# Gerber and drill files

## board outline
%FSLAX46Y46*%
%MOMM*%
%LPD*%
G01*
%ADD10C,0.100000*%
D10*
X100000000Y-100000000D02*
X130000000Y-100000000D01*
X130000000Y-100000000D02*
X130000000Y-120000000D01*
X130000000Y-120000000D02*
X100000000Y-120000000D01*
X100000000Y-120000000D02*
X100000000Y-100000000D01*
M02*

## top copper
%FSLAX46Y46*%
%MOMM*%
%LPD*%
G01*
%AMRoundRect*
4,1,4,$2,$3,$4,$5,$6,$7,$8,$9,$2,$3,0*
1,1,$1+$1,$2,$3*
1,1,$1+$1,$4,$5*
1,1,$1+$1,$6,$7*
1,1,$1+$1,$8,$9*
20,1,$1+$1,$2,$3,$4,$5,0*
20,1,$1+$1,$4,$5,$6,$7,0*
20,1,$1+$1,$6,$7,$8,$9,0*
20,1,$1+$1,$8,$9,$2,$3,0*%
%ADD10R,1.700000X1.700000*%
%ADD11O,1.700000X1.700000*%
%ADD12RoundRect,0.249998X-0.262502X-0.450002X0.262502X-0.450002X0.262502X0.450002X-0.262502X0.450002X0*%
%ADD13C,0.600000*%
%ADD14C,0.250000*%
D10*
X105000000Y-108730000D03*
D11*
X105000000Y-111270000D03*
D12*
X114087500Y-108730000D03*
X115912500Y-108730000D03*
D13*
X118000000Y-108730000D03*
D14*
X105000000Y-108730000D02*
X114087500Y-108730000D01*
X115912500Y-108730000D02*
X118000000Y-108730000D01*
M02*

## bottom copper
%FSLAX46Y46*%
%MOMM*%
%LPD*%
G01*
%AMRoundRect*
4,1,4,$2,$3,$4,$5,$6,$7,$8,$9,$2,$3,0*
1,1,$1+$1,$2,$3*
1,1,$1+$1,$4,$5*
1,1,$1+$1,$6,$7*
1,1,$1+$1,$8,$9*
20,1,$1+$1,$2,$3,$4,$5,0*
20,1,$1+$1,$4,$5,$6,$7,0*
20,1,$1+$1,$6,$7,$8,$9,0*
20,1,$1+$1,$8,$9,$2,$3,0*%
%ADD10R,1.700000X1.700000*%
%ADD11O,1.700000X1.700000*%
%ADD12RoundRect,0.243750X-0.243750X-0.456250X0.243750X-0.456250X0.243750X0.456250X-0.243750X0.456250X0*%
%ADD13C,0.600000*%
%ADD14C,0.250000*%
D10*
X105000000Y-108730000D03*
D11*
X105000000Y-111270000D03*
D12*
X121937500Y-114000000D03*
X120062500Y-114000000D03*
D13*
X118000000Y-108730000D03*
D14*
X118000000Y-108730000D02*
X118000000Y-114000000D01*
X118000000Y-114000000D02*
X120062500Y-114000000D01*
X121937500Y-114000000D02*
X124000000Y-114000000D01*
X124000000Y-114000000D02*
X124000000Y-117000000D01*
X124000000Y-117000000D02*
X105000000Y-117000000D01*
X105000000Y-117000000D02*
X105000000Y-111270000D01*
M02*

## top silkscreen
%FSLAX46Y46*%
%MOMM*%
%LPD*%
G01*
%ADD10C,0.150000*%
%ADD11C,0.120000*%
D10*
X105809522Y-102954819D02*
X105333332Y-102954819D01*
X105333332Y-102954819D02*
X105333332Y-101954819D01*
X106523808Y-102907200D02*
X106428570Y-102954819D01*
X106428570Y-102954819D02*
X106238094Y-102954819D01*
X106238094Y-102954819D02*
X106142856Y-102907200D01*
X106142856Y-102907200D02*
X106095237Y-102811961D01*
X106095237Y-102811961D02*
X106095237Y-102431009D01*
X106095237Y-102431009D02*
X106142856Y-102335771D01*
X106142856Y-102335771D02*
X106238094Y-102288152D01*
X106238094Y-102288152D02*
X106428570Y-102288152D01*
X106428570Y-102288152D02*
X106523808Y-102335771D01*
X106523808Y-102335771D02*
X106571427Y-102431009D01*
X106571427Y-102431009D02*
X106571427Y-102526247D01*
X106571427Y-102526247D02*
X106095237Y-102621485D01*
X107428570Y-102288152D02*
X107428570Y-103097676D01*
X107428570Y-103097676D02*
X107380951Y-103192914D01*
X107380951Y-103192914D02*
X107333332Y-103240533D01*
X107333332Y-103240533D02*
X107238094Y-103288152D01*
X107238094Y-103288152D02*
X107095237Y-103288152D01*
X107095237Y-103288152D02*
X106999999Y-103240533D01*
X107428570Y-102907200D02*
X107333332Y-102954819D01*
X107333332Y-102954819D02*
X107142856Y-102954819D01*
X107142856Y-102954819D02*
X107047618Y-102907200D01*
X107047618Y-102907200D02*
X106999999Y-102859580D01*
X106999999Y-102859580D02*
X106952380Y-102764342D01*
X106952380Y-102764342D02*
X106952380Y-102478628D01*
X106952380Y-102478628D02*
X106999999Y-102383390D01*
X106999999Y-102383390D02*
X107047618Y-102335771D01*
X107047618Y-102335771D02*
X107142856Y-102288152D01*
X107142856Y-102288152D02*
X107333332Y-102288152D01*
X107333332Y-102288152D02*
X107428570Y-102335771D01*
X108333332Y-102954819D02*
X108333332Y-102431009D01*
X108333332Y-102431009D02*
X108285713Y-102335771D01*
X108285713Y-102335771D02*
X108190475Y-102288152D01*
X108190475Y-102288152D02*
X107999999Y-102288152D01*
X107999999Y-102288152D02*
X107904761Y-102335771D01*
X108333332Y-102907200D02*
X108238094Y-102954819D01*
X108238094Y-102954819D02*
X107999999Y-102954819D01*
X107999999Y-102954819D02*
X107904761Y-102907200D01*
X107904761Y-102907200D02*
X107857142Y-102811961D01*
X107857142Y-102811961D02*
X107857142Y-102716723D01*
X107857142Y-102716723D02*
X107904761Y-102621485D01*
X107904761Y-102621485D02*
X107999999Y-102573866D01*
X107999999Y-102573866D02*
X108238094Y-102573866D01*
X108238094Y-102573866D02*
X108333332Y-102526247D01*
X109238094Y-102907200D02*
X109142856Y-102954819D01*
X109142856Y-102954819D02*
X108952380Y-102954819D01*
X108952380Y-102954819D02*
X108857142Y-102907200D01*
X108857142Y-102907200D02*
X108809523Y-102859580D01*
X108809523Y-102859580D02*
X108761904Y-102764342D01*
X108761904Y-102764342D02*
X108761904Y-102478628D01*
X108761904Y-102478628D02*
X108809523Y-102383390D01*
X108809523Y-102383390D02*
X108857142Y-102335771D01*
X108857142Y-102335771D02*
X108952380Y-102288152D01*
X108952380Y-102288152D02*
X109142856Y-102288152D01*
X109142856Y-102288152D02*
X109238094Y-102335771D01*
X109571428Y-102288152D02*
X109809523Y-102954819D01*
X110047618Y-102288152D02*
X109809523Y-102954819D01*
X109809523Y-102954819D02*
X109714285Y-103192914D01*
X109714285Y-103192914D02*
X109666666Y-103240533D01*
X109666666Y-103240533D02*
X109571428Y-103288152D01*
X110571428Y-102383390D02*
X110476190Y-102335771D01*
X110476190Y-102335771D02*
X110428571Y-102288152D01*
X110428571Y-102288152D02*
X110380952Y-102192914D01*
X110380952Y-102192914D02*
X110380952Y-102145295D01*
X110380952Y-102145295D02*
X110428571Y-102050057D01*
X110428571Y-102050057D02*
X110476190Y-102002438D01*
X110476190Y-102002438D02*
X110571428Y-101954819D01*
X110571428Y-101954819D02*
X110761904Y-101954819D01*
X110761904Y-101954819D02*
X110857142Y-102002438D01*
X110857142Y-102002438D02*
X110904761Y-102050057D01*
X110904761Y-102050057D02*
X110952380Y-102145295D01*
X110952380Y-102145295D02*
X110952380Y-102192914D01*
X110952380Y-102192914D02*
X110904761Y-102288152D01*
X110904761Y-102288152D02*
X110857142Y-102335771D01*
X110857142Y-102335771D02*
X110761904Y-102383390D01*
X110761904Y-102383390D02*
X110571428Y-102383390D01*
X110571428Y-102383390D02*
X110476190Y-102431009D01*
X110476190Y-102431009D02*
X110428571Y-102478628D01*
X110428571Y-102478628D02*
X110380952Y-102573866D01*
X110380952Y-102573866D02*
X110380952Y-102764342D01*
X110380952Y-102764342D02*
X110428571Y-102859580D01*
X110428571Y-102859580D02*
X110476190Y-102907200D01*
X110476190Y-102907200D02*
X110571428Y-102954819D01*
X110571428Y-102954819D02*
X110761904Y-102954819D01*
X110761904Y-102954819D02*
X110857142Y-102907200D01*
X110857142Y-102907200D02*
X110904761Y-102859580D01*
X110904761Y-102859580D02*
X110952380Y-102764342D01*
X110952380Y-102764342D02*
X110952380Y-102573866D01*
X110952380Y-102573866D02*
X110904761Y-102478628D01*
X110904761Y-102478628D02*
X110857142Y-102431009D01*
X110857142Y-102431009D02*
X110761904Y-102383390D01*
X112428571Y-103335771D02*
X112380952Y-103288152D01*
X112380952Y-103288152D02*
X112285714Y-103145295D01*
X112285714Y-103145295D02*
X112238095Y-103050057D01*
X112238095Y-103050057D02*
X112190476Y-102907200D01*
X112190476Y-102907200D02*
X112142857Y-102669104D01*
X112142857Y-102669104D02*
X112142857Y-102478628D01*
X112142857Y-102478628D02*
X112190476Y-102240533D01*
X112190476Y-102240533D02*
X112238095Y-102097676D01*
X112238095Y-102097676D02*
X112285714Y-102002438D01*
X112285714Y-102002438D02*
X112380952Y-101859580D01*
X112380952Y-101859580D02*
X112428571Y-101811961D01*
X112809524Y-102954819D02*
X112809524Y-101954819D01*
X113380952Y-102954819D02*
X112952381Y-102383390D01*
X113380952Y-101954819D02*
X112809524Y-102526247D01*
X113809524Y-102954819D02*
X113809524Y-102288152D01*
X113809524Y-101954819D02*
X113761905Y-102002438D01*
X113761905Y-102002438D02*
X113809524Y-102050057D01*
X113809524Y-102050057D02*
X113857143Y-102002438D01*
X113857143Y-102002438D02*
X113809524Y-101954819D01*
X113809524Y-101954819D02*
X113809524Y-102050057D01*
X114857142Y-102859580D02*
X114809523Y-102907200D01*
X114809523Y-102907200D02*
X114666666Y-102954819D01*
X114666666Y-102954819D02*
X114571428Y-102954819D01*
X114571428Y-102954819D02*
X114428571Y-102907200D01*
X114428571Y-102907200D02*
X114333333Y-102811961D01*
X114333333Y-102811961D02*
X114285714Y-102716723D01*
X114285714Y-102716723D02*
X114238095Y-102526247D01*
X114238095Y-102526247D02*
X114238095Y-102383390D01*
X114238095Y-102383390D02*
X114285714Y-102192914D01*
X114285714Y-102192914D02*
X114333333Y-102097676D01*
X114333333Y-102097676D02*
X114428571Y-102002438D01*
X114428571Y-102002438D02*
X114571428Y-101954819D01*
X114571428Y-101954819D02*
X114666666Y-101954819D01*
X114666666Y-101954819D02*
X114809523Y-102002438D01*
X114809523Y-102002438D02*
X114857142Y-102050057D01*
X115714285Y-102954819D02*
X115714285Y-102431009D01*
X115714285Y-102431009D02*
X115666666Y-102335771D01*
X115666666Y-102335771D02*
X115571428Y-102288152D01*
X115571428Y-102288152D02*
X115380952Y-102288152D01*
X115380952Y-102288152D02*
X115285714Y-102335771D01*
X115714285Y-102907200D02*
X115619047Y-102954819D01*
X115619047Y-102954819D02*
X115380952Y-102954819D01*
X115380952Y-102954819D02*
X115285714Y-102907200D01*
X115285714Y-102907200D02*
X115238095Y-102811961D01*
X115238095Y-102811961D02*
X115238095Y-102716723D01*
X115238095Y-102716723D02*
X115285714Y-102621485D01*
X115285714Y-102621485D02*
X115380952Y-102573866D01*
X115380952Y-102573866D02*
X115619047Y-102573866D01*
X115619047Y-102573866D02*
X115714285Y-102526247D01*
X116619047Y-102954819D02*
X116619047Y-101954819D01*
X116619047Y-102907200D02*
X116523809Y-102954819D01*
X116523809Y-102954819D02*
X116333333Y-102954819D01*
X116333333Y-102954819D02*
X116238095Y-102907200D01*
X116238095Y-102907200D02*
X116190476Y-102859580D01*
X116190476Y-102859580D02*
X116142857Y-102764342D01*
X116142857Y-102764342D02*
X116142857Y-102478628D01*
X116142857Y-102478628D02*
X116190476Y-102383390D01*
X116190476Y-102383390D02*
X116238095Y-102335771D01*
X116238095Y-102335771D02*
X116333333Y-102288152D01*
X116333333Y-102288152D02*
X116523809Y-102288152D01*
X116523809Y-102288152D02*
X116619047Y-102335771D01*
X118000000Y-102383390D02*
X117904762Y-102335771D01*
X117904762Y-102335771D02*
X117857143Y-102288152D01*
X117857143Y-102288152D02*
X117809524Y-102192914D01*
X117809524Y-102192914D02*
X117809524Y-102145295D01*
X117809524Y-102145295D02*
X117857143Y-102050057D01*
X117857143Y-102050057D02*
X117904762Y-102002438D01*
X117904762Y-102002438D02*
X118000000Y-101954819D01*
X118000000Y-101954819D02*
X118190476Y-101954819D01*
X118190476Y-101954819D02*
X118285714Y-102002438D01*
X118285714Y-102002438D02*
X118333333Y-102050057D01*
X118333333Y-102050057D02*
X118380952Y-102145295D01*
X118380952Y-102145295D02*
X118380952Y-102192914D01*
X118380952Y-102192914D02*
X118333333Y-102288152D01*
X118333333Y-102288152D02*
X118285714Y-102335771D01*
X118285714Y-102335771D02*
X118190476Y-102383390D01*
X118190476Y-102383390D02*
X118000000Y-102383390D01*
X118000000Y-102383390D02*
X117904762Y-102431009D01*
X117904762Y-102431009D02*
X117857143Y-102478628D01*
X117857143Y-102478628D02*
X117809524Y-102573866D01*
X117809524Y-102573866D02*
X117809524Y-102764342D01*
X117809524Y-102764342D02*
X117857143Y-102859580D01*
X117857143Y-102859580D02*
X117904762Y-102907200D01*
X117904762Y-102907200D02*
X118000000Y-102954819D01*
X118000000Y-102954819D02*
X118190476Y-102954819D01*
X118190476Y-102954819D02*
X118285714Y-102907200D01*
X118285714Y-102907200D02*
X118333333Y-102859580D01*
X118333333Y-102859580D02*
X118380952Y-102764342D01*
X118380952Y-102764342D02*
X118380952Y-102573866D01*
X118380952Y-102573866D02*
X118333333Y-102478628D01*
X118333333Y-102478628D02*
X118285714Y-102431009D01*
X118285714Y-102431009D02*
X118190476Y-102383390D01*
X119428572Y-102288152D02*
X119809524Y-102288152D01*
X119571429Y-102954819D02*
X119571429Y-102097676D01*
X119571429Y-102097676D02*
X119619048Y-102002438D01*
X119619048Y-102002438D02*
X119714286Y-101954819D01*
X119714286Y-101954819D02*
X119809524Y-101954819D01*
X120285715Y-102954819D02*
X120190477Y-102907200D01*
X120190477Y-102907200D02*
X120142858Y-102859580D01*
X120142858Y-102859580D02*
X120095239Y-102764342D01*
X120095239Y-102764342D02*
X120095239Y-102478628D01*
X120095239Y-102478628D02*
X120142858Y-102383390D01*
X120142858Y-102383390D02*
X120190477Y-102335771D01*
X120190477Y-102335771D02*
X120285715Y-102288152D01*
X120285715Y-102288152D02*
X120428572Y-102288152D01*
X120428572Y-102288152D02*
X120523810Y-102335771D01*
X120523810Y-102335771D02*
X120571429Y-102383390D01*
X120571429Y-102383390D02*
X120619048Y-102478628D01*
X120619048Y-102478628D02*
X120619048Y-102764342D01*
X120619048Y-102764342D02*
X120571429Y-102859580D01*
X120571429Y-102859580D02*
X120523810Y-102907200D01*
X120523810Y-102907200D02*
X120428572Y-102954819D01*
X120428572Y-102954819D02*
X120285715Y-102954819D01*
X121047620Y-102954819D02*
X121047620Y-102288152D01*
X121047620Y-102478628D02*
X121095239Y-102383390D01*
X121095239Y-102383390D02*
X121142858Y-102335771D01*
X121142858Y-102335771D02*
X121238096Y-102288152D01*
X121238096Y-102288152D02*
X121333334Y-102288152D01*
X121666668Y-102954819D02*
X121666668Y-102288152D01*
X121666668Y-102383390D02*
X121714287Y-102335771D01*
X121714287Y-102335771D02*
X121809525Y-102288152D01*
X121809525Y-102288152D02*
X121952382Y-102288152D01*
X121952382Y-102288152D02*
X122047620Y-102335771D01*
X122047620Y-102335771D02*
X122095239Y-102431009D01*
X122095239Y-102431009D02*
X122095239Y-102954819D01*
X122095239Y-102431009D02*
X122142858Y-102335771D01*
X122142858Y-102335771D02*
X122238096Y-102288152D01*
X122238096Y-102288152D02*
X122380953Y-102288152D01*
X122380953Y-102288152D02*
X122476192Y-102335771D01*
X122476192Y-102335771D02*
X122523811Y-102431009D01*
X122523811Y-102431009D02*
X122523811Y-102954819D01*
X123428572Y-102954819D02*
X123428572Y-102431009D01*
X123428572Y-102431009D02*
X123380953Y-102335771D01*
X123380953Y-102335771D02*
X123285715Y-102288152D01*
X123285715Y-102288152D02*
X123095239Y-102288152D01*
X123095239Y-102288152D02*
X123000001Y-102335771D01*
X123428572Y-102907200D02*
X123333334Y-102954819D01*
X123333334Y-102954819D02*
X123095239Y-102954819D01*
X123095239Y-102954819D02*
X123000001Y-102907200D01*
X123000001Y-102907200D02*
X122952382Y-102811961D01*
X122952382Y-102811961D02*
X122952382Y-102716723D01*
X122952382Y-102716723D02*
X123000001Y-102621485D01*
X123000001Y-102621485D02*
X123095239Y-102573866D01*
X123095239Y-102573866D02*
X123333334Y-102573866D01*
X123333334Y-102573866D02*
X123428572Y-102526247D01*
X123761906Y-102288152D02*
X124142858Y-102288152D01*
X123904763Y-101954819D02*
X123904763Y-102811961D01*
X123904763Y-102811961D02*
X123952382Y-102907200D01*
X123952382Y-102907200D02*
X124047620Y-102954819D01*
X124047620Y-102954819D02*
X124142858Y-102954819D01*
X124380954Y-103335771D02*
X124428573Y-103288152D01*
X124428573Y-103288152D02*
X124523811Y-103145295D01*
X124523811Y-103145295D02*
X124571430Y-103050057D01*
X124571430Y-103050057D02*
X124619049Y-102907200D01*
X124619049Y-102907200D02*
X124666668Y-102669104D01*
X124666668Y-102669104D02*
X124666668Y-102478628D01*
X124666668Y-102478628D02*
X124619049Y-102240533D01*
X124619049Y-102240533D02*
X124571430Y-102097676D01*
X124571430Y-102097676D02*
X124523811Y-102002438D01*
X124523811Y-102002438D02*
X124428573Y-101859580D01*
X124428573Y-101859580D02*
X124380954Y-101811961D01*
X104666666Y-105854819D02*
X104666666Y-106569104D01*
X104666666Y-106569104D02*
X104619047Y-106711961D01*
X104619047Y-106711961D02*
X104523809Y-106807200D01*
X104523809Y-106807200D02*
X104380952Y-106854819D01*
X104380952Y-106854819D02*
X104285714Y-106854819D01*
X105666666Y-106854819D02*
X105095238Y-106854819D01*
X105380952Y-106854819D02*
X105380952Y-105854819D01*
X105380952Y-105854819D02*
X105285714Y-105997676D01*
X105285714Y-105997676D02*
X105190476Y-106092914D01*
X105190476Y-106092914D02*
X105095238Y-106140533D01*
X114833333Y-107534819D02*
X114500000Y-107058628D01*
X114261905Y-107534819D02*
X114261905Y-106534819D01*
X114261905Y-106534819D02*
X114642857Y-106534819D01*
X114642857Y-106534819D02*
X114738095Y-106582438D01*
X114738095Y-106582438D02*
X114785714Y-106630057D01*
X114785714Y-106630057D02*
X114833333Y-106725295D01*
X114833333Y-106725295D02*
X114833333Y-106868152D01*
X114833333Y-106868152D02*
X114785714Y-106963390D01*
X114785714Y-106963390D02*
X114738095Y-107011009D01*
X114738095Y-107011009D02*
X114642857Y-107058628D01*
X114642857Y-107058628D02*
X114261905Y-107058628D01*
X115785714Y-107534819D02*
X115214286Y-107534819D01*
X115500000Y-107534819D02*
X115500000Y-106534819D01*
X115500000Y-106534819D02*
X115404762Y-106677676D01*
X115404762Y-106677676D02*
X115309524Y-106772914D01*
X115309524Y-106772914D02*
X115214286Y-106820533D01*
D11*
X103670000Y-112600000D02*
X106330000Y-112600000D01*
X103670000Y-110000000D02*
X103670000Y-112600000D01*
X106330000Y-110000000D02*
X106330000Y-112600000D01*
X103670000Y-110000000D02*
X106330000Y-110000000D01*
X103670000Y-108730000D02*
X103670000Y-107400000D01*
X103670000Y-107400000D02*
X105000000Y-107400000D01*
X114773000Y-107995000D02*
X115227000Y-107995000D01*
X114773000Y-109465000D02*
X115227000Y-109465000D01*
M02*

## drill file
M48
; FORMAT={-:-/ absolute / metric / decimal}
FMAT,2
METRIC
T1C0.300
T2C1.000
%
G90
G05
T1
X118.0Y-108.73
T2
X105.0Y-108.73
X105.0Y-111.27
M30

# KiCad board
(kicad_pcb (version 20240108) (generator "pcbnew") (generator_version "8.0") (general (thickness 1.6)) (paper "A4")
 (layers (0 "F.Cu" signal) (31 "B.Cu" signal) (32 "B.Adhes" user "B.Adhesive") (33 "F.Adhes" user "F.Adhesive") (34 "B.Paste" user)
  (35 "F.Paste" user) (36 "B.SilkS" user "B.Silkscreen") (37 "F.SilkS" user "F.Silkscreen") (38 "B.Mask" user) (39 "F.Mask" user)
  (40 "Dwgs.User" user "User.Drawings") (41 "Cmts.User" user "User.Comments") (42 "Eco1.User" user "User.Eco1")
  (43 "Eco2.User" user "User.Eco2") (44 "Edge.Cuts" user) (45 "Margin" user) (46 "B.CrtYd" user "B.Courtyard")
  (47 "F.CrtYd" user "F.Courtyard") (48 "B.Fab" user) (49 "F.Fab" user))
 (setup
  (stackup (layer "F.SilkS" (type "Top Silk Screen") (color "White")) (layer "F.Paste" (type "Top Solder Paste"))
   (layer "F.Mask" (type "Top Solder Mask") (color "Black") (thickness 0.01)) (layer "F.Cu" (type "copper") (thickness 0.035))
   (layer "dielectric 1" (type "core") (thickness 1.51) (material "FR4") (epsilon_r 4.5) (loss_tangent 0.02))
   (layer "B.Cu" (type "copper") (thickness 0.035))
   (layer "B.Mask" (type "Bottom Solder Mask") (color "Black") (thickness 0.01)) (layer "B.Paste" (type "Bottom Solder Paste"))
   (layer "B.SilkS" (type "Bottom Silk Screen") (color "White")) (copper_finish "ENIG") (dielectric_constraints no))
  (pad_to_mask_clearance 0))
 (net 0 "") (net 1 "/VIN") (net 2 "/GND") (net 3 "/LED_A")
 (gr_line (start 100 100) (end 130 100) (stroke (width 0.1) (type default)) (layer "Edge.Cuts"))
 (gr_line (start 130 100) (end 130 120) (stroke (width 0.1) (type default)) (layer "Edge.Cuts"))
 (gr_line (start 130 120) (end 100 120) (stroke (width 0.1) (type default)) (layer "Edge.Cuts"))
 (gr_line (start 100 120) (end 100 100) (stroke (width 0.1) (type default)) (layer "Edge.Cuts"))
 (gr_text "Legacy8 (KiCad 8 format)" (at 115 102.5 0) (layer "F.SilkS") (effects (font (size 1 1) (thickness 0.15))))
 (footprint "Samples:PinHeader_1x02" (layer "F.Cu") (at 105 108.73)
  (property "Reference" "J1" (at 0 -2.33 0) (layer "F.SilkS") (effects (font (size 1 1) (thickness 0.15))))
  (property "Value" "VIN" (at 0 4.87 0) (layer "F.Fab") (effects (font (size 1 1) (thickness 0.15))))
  (fp_line (start -1.33 3.87) (end 1.33 3.87) (stroke (width 0.12) (type solid)) (layer "F.SilkS"))
  (fp_line (start -1.33 1.27) (end -1.33 3.87) (stroke (width 0.12) (type solid)) (layer "F.SilkS"))
  (fp_line (start 1.33 1.27) (end 1.33 3.87) (stroke (width 0.12) (type solid)) (layer "F.SilkS"))
  (fp_line (start -1.33 1.27) (end 1.33 1.27) (stroke (width 0.12) (type solid)) (layer "F.SilkS"))
  (fp_line (start -1.33 0) (end -1.33 -1.33) (stroke (width 0.12) (type solid)) (layer "F.SilkS"))
  (fp_line (start -1.33 -1.33) (end 0 -1.33) (stroke (width 0.12) (type solid)) (layer "F.SilkS"))
  (pad "1" thru_hole rect (at 0 0) (size 1.7 1.7) (drill 1) (layers "*.Cu" "*.Mask") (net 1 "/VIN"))
  (pad "2" thru_hole oval (at 0 2.54) (size 1.7 1.7) (drill 1) (layers "*.Cu" "*.Mask") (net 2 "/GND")))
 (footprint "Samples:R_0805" (layer "F.Cu") (at 115 108.73)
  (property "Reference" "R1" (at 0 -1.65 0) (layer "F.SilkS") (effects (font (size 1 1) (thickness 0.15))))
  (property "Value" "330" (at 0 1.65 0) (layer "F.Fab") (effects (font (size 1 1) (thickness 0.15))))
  (fp_line (start -0.227 -0.735) (end 0.227 -0.735) (stroke (width 0.12) (type solid)) (layer "F.SilkS"))
  (fp_line (start -0.227 0.735) (end 0.227 0.735) (stroke (width 0.12) (type solid)) (layer "F.SilkS"))
  (pad "1" smd roundrect (at -0.9125 0) (size 1.025 1.4) (layers "F.Cu" "F.Paste" "F.Mask") (roundrect_rratio 0.2439) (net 1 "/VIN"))
  (pad "2" smd roundrect (at 0.9125 0) (size 1.025 1.4) (layers "F.Cu" "F.Paste" "F.Mask") (roundrect_rratio 0.2439) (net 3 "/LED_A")))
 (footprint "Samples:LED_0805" (layer "B.Cu") (at 121 114)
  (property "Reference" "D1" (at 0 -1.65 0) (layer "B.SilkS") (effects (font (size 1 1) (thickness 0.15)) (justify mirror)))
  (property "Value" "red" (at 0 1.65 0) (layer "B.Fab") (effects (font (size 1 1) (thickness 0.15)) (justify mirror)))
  (pad "1" smd roundrect (at 0.9375 0) (size 0.975 1.4) (layers "B.Cu" "B.Paste" "B.Mask") (roundrect_rratio 0.25) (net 2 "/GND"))
  (pad "2" smd roundrect (at -0.9375 0) (size 0.975 1.4) (layers "B.Cu" "B.Paste" "B.Mask") (roundrect_rratio 0.25) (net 3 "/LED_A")))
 (segment (start 105 108.73) (end 114.0875 108.73) (width 0.25) (layer "F.Cu") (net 1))
 (segment (start 115.9125 108.73) (end 118 108.73) (width 0.25) (layer "F.Cu") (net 3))
 (segment (start 118 108.73) (end 118 114) (width 0.25) (layer "B.Cu") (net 3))
 (segment (start 118 114) (end 120.0625 114) (width 0.25) (layer "B.Cu") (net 3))
 (segment (start 121.9375 114) (end 124 114) (width 0.25) (layer "B.Cu") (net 2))
 (segment (start 124 114) (end 124 117) (width 0.25) (layer "B.Cu") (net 2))
 (segment (start 124 117) (end 105 117) (width 0.25) (layer "B.Cu") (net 2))
 (segment (start 105 117) (end 105 111.27) (width 0.25) (layer "B.Cu") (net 2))
 (via (at 118 108.73) (size 0.6) (drill 0.3) (layers "F.Cu" "B.Cu") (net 3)))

